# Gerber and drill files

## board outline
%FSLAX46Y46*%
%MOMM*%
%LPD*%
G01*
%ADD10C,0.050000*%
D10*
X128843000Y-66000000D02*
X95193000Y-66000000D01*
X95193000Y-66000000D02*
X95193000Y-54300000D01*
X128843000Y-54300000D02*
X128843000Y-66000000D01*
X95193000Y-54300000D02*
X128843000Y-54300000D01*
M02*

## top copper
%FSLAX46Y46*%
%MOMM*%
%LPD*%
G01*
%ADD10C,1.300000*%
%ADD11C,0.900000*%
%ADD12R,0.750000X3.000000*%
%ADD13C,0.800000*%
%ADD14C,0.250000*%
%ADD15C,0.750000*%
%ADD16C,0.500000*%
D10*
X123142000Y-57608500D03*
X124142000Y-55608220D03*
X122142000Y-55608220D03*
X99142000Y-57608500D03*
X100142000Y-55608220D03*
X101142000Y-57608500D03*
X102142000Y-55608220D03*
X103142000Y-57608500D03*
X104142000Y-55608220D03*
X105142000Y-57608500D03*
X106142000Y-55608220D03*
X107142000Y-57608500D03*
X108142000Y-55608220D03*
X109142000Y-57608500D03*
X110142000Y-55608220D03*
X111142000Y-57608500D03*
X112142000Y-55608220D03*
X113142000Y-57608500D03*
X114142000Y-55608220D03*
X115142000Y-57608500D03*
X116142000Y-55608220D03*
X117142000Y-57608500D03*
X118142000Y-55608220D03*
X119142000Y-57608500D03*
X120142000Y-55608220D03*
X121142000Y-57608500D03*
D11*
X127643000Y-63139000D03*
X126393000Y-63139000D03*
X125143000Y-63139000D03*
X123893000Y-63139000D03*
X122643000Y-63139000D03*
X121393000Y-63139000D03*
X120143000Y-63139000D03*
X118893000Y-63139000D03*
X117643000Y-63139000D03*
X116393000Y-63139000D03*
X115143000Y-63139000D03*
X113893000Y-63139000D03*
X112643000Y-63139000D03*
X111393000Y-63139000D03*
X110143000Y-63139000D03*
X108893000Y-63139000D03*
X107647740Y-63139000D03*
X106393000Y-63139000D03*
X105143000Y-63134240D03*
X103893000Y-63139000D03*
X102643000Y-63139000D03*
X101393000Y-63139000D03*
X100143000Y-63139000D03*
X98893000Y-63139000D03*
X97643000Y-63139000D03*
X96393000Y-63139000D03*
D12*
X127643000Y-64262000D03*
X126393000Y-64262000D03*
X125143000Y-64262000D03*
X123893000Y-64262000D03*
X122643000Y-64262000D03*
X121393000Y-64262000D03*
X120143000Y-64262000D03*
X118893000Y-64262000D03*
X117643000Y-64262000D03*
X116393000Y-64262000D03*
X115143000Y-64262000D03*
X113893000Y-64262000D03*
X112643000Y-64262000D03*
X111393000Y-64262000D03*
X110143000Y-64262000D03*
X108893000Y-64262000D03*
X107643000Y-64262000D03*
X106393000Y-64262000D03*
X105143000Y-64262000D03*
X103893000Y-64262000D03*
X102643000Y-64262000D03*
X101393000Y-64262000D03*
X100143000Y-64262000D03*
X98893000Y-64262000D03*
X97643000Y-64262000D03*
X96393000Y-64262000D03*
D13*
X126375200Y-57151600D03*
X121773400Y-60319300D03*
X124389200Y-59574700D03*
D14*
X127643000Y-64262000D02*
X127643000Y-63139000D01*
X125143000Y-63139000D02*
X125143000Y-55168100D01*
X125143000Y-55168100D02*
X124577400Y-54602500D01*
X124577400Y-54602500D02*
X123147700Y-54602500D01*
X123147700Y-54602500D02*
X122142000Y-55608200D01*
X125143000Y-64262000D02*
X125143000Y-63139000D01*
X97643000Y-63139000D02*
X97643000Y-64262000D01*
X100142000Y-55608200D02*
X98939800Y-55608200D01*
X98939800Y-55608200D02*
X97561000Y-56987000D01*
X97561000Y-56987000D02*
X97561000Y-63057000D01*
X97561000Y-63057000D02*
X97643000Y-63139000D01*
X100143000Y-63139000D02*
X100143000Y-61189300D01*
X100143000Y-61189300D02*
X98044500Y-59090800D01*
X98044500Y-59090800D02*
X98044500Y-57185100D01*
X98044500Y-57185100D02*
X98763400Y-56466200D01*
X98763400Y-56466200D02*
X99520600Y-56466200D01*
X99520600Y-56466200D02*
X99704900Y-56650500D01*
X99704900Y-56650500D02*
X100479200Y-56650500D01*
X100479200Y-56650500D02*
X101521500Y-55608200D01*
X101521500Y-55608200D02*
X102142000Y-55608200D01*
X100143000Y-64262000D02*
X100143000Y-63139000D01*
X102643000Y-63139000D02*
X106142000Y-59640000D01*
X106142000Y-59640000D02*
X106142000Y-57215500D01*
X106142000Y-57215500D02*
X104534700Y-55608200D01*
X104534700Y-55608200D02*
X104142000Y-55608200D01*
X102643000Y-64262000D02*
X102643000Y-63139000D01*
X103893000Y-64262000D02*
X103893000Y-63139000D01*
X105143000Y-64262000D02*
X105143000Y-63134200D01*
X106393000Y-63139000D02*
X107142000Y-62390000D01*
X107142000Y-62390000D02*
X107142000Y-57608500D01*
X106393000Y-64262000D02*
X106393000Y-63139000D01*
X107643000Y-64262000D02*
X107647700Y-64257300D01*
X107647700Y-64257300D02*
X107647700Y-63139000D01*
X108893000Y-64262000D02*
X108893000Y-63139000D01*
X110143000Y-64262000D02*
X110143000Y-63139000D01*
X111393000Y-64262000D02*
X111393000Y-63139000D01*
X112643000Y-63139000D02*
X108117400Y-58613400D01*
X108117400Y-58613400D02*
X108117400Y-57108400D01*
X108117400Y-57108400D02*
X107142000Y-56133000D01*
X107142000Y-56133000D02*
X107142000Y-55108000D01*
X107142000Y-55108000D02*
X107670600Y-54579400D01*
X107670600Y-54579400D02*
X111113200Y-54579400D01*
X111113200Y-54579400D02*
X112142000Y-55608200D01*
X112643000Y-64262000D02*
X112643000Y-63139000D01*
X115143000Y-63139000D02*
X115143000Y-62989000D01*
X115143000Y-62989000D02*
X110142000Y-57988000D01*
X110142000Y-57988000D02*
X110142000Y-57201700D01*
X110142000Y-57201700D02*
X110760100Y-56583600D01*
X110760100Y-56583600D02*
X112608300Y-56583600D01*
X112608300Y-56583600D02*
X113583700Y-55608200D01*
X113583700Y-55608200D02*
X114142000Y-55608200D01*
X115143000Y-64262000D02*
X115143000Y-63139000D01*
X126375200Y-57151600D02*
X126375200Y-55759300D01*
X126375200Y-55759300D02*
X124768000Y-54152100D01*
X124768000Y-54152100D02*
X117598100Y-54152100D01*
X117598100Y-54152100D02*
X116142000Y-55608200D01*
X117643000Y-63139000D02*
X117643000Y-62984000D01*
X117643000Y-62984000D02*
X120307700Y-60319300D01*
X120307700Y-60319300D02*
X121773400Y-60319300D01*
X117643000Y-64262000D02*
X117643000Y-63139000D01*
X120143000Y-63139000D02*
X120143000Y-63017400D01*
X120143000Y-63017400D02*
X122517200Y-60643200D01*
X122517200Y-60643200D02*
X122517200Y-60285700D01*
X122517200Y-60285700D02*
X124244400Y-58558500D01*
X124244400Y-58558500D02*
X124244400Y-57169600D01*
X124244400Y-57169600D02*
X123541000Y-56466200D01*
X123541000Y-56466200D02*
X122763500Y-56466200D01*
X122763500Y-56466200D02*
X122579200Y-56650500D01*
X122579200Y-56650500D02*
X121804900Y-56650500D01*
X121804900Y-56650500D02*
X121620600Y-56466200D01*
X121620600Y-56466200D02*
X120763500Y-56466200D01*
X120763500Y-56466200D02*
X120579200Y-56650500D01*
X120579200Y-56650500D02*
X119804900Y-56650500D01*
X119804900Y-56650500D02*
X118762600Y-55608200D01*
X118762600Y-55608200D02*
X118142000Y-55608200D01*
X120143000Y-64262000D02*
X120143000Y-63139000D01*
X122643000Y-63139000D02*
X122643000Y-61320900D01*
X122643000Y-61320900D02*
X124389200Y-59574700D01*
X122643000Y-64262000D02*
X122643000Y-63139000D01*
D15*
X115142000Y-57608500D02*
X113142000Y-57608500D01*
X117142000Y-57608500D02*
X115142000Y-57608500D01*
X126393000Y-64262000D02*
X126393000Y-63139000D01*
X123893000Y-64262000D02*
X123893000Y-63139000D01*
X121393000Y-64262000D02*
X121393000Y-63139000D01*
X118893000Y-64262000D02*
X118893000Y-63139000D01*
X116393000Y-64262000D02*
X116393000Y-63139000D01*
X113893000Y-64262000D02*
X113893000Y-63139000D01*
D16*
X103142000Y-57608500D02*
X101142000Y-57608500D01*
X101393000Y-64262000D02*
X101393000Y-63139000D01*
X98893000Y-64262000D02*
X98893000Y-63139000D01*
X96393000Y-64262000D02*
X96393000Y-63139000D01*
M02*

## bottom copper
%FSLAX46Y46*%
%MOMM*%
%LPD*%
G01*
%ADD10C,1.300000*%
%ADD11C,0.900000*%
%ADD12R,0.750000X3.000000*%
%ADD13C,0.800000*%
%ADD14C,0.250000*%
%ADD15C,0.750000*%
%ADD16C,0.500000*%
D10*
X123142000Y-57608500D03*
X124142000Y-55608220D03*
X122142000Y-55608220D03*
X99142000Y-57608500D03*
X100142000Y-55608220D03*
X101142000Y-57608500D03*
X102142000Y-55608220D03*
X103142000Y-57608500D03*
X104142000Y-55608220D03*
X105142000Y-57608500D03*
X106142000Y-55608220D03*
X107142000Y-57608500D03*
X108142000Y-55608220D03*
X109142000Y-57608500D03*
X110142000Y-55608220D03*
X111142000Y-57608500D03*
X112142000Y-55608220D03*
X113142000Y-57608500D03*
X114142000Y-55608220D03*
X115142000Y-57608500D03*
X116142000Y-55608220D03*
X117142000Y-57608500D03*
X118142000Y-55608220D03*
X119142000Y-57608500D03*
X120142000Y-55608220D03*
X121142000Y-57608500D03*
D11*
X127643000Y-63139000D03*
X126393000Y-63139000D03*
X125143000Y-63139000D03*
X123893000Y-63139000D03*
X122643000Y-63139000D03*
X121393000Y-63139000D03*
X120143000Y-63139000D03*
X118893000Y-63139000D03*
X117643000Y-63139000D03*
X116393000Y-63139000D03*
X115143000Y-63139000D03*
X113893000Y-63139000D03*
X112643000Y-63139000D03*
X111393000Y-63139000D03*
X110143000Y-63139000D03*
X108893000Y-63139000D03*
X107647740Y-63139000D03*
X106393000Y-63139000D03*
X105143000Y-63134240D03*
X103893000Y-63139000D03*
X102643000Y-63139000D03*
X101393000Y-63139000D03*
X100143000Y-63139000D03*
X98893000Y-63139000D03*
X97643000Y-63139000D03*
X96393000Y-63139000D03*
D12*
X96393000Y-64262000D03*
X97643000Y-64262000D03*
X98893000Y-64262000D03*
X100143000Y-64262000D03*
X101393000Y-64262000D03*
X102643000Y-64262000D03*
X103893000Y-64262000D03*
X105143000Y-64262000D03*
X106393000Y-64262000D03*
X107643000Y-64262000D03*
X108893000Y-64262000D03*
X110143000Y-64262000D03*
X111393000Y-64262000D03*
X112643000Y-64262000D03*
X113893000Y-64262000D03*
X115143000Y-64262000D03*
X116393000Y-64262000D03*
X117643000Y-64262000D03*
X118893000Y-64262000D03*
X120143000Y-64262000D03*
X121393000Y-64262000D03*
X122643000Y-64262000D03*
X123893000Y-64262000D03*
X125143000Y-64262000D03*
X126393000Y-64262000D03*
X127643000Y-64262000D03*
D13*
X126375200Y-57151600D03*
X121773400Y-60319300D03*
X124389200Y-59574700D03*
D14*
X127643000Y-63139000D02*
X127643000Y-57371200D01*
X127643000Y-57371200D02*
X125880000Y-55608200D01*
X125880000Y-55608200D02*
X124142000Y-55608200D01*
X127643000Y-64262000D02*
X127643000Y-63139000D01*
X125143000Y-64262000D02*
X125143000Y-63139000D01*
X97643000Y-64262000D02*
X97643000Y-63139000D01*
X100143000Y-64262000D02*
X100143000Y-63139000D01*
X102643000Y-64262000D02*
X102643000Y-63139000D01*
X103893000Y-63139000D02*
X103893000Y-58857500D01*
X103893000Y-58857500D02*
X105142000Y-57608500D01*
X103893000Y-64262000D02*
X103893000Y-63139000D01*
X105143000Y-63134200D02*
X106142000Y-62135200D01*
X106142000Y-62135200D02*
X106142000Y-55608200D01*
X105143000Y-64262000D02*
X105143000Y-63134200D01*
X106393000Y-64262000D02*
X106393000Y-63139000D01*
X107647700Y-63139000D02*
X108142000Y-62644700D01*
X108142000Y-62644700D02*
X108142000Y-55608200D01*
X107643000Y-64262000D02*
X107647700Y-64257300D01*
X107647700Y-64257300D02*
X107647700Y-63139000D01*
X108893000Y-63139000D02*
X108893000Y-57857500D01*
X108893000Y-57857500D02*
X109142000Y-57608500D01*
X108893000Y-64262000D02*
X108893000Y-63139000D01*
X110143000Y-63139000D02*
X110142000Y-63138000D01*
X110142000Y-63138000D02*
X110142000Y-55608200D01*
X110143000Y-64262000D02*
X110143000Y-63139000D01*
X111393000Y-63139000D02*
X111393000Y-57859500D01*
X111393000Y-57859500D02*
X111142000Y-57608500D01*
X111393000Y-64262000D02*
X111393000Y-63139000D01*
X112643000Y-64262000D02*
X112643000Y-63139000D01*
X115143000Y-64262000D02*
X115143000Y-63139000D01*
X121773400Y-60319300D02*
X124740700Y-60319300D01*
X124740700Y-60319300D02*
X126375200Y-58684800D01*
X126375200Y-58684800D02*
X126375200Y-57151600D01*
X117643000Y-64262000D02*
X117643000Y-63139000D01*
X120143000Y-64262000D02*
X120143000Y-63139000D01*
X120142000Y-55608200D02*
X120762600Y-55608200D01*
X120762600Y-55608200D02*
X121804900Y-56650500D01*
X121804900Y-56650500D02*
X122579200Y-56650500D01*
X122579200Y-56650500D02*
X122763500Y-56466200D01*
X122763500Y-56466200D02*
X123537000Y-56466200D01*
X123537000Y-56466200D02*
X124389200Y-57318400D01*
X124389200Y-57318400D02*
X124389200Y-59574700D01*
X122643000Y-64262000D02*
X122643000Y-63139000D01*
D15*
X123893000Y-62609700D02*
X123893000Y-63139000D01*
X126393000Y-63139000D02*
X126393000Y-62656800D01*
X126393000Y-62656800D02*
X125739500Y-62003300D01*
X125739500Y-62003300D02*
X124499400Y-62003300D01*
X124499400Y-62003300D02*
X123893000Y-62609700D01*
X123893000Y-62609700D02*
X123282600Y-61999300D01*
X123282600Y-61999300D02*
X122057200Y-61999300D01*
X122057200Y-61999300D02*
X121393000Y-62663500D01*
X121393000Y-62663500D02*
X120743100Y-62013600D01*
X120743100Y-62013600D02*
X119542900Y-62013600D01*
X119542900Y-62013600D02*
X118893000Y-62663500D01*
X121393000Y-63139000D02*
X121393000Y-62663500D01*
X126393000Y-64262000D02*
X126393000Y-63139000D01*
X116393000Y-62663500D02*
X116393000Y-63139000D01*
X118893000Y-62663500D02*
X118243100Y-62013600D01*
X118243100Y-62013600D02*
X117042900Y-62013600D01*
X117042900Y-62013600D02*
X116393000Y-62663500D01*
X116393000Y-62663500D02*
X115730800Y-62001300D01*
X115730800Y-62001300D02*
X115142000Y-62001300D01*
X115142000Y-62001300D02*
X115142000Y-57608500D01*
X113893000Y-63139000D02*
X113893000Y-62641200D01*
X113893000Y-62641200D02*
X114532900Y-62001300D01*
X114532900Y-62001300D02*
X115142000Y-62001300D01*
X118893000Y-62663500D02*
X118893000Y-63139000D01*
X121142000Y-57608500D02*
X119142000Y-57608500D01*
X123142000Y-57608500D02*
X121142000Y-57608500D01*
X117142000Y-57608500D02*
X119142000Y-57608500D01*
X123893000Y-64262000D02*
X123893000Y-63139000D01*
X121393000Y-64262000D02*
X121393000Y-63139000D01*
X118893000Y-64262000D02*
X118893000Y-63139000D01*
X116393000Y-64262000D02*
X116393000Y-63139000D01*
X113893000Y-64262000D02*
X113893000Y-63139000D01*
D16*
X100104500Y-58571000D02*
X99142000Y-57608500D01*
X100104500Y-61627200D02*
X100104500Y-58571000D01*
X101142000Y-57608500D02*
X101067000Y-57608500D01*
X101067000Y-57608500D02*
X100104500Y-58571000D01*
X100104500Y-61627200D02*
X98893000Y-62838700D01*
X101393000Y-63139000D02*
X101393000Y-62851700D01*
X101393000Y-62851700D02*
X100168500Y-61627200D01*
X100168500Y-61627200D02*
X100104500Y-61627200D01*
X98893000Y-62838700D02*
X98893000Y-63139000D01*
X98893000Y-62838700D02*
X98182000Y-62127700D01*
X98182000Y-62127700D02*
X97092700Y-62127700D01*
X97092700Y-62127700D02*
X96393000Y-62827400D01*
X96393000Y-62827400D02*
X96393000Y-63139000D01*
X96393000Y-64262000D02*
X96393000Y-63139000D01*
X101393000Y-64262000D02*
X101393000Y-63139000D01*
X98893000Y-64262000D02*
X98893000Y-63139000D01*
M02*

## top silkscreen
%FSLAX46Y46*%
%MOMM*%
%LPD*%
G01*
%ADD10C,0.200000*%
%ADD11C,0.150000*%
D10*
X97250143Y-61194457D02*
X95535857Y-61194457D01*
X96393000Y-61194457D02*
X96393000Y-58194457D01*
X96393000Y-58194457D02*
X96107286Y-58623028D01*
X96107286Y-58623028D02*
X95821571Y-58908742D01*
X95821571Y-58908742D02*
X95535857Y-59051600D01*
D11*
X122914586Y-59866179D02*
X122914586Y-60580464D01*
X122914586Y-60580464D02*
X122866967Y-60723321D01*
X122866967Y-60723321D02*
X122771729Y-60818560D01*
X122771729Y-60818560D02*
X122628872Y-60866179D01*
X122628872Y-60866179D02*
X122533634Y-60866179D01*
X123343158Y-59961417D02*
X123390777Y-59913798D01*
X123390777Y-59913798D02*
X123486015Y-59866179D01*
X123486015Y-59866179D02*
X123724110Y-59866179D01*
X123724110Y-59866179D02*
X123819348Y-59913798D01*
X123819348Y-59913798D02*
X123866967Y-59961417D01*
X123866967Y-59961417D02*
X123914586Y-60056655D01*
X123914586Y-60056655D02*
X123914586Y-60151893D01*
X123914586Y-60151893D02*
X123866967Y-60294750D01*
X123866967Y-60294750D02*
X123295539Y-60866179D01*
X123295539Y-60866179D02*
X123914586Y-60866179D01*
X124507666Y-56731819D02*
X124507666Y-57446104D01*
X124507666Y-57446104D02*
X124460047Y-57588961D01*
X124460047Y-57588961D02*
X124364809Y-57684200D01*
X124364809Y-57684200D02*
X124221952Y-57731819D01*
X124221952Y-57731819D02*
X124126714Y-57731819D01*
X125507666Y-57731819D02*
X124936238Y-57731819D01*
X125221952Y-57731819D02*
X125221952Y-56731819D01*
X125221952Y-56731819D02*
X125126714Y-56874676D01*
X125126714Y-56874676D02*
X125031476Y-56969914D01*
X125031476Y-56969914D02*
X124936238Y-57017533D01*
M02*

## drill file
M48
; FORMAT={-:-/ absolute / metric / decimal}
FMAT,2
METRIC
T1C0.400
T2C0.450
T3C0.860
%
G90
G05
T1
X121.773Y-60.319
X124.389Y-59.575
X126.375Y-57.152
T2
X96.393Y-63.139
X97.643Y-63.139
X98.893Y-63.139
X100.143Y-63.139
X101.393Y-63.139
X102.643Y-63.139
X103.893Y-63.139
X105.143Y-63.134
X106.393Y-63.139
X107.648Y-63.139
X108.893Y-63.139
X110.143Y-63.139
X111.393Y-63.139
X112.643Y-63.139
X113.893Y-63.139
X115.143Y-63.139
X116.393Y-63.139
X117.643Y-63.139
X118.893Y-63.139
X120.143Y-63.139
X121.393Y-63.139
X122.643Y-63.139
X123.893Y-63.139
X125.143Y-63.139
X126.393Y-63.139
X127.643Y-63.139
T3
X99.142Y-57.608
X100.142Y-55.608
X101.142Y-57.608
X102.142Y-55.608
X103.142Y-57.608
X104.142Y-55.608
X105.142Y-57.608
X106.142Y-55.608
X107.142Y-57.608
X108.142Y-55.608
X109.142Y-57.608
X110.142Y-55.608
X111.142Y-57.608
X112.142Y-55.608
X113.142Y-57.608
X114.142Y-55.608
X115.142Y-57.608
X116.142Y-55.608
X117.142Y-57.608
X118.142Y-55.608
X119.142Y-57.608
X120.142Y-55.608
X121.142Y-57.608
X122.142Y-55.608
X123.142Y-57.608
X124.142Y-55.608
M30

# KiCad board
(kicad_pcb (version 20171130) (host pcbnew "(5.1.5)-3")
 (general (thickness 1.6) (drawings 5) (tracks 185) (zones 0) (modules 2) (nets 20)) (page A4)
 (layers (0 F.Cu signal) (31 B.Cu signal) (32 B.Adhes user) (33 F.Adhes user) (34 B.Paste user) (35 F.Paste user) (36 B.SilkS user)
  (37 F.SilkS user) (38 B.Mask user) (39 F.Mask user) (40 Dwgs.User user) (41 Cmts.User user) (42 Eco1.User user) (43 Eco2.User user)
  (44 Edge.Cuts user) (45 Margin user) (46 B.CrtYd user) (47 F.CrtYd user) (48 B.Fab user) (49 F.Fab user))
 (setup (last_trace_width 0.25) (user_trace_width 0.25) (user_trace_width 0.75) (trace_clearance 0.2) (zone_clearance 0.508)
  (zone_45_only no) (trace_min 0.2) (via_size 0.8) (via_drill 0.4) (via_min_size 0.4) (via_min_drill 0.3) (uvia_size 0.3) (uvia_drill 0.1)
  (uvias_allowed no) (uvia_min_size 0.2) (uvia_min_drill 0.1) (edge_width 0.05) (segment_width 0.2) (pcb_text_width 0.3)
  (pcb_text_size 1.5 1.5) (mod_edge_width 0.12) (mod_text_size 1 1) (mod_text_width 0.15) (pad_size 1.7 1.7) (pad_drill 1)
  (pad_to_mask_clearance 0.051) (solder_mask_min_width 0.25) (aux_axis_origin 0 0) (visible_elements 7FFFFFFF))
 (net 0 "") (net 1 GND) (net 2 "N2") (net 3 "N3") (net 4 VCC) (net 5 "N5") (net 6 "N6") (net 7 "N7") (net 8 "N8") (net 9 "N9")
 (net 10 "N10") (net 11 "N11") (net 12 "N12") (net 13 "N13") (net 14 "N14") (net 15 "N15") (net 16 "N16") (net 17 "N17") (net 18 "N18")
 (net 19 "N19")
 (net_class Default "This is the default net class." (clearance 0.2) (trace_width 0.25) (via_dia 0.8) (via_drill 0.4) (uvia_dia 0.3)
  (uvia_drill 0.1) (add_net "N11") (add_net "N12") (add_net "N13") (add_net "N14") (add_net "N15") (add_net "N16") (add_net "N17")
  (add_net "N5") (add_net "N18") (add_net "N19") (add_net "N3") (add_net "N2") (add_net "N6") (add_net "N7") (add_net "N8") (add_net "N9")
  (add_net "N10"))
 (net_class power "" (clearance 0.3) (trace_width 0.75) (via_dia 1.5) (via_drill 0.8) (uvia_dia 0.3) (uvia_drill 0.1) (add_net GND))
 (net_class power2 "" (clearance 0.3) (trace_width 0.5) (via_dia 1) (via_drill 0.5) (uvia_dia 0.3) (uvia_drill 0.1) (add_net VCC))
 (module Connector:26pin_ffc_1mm (layer F.Cu) (at 124.142 52.8955 180)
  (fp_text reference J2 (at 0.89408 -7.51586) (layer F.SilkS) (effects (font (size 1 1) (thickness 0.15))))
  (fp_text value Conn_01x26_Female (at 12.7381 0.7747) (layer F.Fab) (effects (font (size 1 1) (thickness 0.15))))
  (pad 25 thru_hole circle (at 1 -4.713 180) (size 1.3 1.3) (drill 0.86) (layers *.Cu *.Mask) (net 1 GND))
  (pad 26 thru_hole circle (at 0 -2.71272 180) (size 1.3 1.3) (drill 0.86) (layers *.Cu *.Mask) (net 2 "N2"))
  (pad 24 thru_hole circle (at 2 -2.71272 180) (size 1.3 1.3) (drill 0.86) (layers *.Cu *.Mask) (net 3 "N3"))
  (pad 1 thru_hole circle (at 25 -4.713 180) (size 1.3 1.3) (drill 0.86) (layers *.Cu *.Mask) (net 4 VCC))
  (pad 2 thru_hole circle (at 24 -2.71272 180) (size 1.3 1.3) (drill 0.86) (layers *.Cu *.Mask) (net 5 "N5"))
  (pad 3 thru_hole circle (at 23 -4.713 180) (size 1.3 1.3) (drill 0.86) (layers *.Cu *.Mask) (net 4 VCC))
  (pad 4 thru_hole circle (at 22 -2.71272 180) (size 1.3 1.3) (drill 0.86) (layers *.Cu *.Mask) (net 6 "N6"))
  (pad 5 thru_hole circle (at 21 -4.713 180) (size 1.3 1.3) (drill 0.86) (layers *.Cu *.Mask) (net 4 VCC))
  (pad 6 thru_hole circle (at 20 -2.71272 180) (size 1.3 1.3) (drill 0.86) (layers *.Cu *.Mask) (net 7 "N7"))
  (pad 7 thru_hole circle (at 19 -4.713 180) (size 1.3 1.3) (drill 0.86) (layers *.Cu *.Mask) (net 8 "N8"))
  (pad 8 thru_hole circle (at 18 -2.71272 180) (size 1.3 1.3) (drill 0.86) (layers *.Cu *.Mask) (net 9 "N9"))
  (pad 9 thru_hole circle (at 17 -4.713 180) (size 1.3 1.3) (drill 0.86) (layers *.Cu *.Mask) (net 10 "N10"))
  (pad 10 thru_hole circle (at 16 -2.71272 180) (size 1.3 1.3) (drill 0.86) (layers *.Cu *.Mask) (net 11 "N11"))
  (pad 11 thru_hole circle (at 15 -4.713 180) (size 1.3 1.3) (drill 0.86) (layers *.Cu *.Mask) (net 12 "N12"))
  (pad 12 thru_hole circle (at 14 -2.71272 180) (size 1.3 1.3) (drill 0.86) (layers *.Cu *.Mask) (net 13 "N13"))
  (pad 13 thru_hole circle (at 13 -4.713 180) (size 1.3 1.3) (drill 0.86) (layers *.Cu *.Mask) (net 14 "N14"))
  (pad 14 thru_hole circle (at 12 -2.71272 180) (size 1.3 1.3) (drill 0.86) (layers *.Cu *.Mask) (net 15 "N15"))
  (pad 15 thru_hole circle (at 11 -4.713 180) (size 1.3 1.3) (drill 0.86) (layers *.Cu *.Mask) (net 1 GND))
  (pad 16 thru_hole circle (at 10 -2.71272 180) (size 1.3 1.3) (drill 0.86) (layers *.Cu *.Mask) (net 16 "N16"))
  (pad 17 thru_hole circle (at 9 -4.713 180) (size 1.3 1.3) (drill 0.86) (layers *.Cu *.Mask) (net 1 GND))
  (pad 18 thru_hole circle (at 8 -2.71272 180) (size 1.3 1.3) (drill 0.86) (layers *.Cu *.Mask) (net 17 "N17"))
  (pad 19 thru_hole circle (at 7 -4.713 180) (size 1.3 1.3) (drill 0.86) (layers *.Cu *.Mask) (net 1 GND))
  (pad 20 thru_hole circle (at 6 -2.71272 180) (size 1.3 1.3) (drill 0.86) (layers *.Cu *.Mask) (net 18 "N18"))
  (pad 21 thru_hole circle (at 5 -4.713 180) (size 1.3 1.3) (drill 0.86) (layers *.Cu *.Mask) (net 1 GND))
  (pad 22 thru_hole circle (at 4 -2.71272 180) (size 1.3 1.3) (drill 0.86) (layers *.Cu *.Mask) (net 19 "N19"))
  (pad 23 thru_hole circle (at 3 -4.713 180) (size 1.3 1.3) (drill 0.86) (layers *.Cu *.Mask) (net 1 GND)))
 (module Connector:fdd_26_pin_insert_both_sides (layer F.Cu) (at 96.393 64.389)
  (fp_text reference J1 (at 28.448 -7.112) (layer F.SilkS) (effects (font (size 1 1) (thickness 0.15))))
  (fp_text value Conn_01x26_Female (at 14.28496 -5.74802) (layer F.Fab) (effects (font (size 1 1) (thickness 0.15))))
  (pad 26 thru_hole circle (at 31.25 -1.25) (size 0.9 0.9) (drill 0.45) (layers *.Cu *.Mask) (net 2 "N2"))
  (pad 25 thru_hole circle (at 30 -1.25) (size 0.9 0.9) (drill 0.45) (layers *.Cu *.Mask) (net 1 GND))
  (pad 24 thru_hole circle (at 28.75 -1.25) (size 0.9 0.9) (drill 0.45) (layers *.Cu *.Mask) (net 3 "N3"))
  (pad 23 thru_hole circle (at 27.5 -1.25) (size 0.9 0.9) (drill 0.45) (layers *.Cu *.Mask) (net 1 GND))
  (pad 22 thru_hole circle (at 26.25 -1.25) (size 0.9 0.9) (drill 0.45) (layers *.Cu *.Mask) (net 19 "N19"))
  (pad 21 thru_hole circle (at 25 -1.25) (size 0.9 0.9) (drill 0.45) (layers *.Cu *.Mask) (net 1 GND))
  (pad 20 thru_hole circle (at 23.75 -1.25) (size 0.9 0.9) (drill 0.45) (layers *.Cu *.Mask) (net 18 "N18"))
  (pad 19 thru_hole circle (at 22.5 -1.25) (size 0.9 0.9) (drill 0.45) (layers *.Cu *.Mask) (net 1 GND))
  (pad 18 thru_hole circle (at 21.25 -1.25) (size 0.9 0.9) (drill 0.45) (layers *.Cu *.Mask) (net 17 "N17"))
  (pad 17 thru_hole circle (at 20 -1.25) (size 0.9 0.9) (drill 0.45) (layers *.Cu *.Mask) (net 1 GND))
  (pad 16 thru_hole circle (at 18.75 -1.25) (size 0.9 0.9) (drill 0.45) (layers *.Cu *.Mask) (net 16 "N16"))
  (pad 15 thru_hole circle (at 17.5 -1.25 90) (size 0.9 0.9) (drill 0.45) (layers *.Cu *.Mask) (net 1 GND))
  (pad 14 thru_hole circle (at 16.25 -1.25) (size 0.9 0.9) (drill 0.45) (layers *.Cu *.Mask) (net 15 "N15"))
  (pad 13 thru_hole circle (at 15 -1.25) (size 0.9 0.9) (drill 0.45) (layers *.Cu *.Mask) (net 14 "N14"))
  (pad 12 thru_hole circle (at 13.75 -1.25) (size 0.9 0.9) (drill 0.45) (layers *.Cu *.Mask) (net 13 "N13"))
  (pad 11 thru_hole circle (at 12.5 -1.25) (size 0.9 0.9) (drill 0.45) (layers *.Cu *.Mask) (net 12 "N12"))
  (pad 10 thru_hole circle (at 11.25474 -1.25) (size 0.9 0.9) (drill 0.45) (layers *.Cu *.Mask) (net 11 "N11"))
  (pad 9 thru_hole circle (at 10 -1.25) (size 0.9 0.9) (drill 0.45) (layers *.Cu *.Mask) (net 10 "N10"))
  (pad 8 thru_hole circle (at 8.75 -1.25476) (size 0.9 0.9) (drill 0.45) (layers *.Cu *.Mask) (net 9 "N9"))
  (pad 7 thru_hole circle (at 7.5 -1.25) (size 0.9 0.9) (drill 0.45) (layers *.Cu *.Mask) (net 8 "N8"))
  (pad 6 thru_hole circle (at 6.25 -1.25) (size 0.9 0.9) (drill 0.45) (layers *.Cu *.Mask) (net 7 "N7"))
  (pad 5 thru_hole circle (at 5 -1.25) (size 0.9 0.9) (drill 0.45) (layers *.Cu *.Mask) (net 4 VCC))
  (pad 4 thru_hole circle (at 3.75 -1.25) (size 0.9 0.9) (drill 0.45) (layers *.Cu *.Mask) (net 6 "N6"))
  (pad 3 thru_hole circle (at 2.5 -1.25) (size 0.9 0.9) (drill 0.45) (layers *.Cu *.Mask) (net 4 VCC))
  (pad 2 thru_hole circle (at 1.25 -1.25 90) (size 0.9 0.9) (drill 0.45) (layers *.Cu *.Mask) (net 5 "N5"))
  (pad 1 thru_hole circle (at 0 -1.25) (size 0.9 0.9) (drill 0.45) (layers *.Cu *.Mask) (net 4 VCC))
  (pad 26 connect rect (at 31.25 -0.127) (size 0.75 3) (layers F.Cu B.Mask) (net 2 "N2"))
  (pad 25 connect rect (at 30 -0.127) (size 0.75 3) (layers F.Cu B.Mask) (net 1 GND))
  (pad 24 connect rect (at 28.75 -0.127) (size 0.75 3) (layers F.Cu B.Mask) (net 3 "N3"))
  (pad 23 connect rect (at 27.5 -0.127) (size 0.75 3) (layers F.Cu B.Mask) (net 1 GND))
  (pad 22 connect rect (at 26.25 -0.127) (size 0.75 3) (layers F.Cu B.Mask) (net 19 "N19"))
  (pad 21 connect rect (at 25 -0.127) (size 0.75 3) (layers F.Cu B.Mask) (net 1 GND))
  (pad 20 connect rect (at 23.75 -0.127) (size 0.75 3) (layers F.Cu B.Mask) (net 18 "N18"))
  (pad 19 connect rect (at 22.5 -0.127) (size 0.75 3) (layers F.Cu B.Mask) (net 1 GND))
  (pad 18 connect rect (at 21.25 -0.127) (size 0.75 3) (layers F.Cu B.Mask) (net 17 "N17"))
  (pad 17 connect rect (at 20 -0.127) (size 0.75 3) (layers F.Cu B.Mask) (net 1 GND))
  (pad 16 connect rect (at 18.75 -0.127) (size 0.75 3) (layers F.Cu B.Mask) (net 16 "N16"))
  (pad 15 connect rect (at 17.5 -0.127) (size 0.75 3) (layers F.Cu B.Mask) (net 1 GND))
  (pad 14 connect rect (at 16.25 -0.127) (size 0.75 3) (layers F.Cu B.Mask) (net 15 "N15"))
  (pad 13 connect rect (at 15 -0.127) (size 0.75 3) (layers F.Cu B.Mask) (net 14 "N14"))
  (pad 12 connect rect (at 13.75 -0.127) (size 0.75 3) (layers F.Cu B.Mask) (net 13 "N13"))
  (pad 11 connect rect (at 12.5 -0.127) (size 0.75 3) (layers F.Cu B.Mask) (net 12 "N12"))
  (pad 10 connect rect (at 11.25 -0.127) (size 0.75 3) (layers F.Cu B.Mask) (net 11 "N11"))
  (pad 9 connect rect (at 10 -0.127) (size 0.75 3) (layers F.Cu B.Mask) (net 10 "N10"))
  (pad 8 connect rect (at 8.75 -0.127) (size 0.75 3) (layers F.Cu B.Mask) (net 9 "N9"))
  (pad 7 connect rect (at 7.5 -0.127) (size 0.75 3) (layers F.Cu B.Mask) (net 8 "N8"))
  (pad 6 connect rect (at 6.25 -0.127) (size 0.75 3) (layers F.Cu B.Mask) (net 7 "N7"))
  (pad 5 connect rect (at 5 -0.127) (size 0.75 3) (layers F.Cu B.Mask) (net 4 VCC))
  (pad 4 connect rect (at 3.75 -0.127) (size 0.75 3) (layers F.Cu B.Mask) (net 6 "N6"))
  (pad 3 connect rect (at 2.5 -0.127) (size 0.75 3) (layers F.Cu B.Mask) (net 4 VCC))
  (pad 2 connect rect (at 1.25 -0.127) (size 0.75 3) (layers F.Cu B.Mask) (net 5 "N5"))
  (pad 1 connect rect (at 0 -0.127) (size 0.75 3) (layers F.Cu B.Mask) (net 4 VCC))
  (pad 1 connect rect (at 0 -0.127) (size 0.75 3) (layers B.Cu B.Mask) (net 4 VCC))
  (pad 2 connect rect (at 1.25 -0.127) (size 0.75 3) (layers B.Cu B.Mask) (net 5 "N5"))
  (pad 3 connect rect (at 2.5 -0.127) (size 0.75 3) (layers B.Cu B.Mask) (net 4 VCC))
  (pad 4 connect rect (at 3.75 -0.127) (size 0.75 3) (layers B.Cu B.Mask) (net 6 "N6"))
  (pad 5 connect rect (at 5 -0.127) (size 0.75 3) (layers B.Cu B.Mask) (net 4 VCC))
  (pad 6 connect rect (at 6.25 -0.127) (size 0.75 3) (layers B.Cu B.Mask) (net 7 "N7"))
  (pad 7 connect rect (at 7.5 -0.127) (size 0.75 3) (layers B.Cu B.Mask) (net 8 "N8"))
  (pad 8 connect rect (at 8.75 -0.127) (size 0.75 3) (layers B.Cu B.Mask) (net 9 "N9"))
  (pad 9 connect rect (at 10 -0.127) (size 0.75 3) (layers B.Cu B.Mask) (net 10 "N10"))
  (pad 10 connect rect (at 11.25 -0.127) (size 0.75 3) (layers B.Cu B.Mask) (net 11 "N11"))
  (pad 11 connect rect (at 12.5 -0.127) (size 0.75 3) (layers B.Cu B.Mask) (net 12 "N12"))
  (pad 12 connect rect (at 13.75 -0.127) (size 0.75 3) (layers B.Cu B.Mask) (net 13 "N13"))
  (pad 13 connect rect (at 15 -0.127) (size 0.75 3) (layers B.Cu B.Mask) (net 14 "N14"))
  (pad 14 connect rect (at 16.25 -0.127) (size 0.75 3) (layers B.Cu B.Mask) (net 15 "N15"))
  (pad 15 connect rect (at 17.5 -0.127) (size 0.75 3) (layers B.Cu B.Mask) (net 1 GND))
  (pad 16 connect rect (at 18.75 -0.127) (size 0.75 3) (layers B.Cu B.Mask) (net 16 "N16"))
  (pad 17 connect rect (at 20 -0.127) (size 0.75 3) (layers B.Cu B.Mask) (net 1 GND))
  (pad 18 connect rect (at 21.25 -0.127) (size 0.75 3) (layers B.Cu B.Mask) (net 17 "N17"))
  (pad 19 connect rect (at 22.5 -0.127) (size 0.75 3) (layers B.Cu B.Mask) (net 1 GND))
  (pad 20 connect rect (at 23.75 -0.127) (size 0.75 3) (layers B.Cu B.Mask) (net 18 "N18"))
  (pad 21 connect rect (at 25 -0.127) (size 0.75 3) (layers B.Cu B.Mask) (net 1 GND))
  (pad 22 connect rect (at 26.25 -0.127) (size 0.75 3) (layers B.Cu B.Mask) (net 19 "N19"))
  (pad 23 connect rect (at 27.5 -0.127) (size 0.75 3) (layers B.Cu B.Mask) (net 1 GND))
  (pad 24 connect rect (at 28.75 -0.127) (size 0.75 3) (layers B.Cu B.Mask) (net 3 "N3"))
  (pad 25 connect rect (at 30 -0.127) (size 0.75 3) (layers B.Cu B.Mask) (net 1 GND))
  (pad 26 connect rect (at 31.25 -0.127) (size 0.75 3) (layers B.Cu B.Mask) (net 2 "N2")))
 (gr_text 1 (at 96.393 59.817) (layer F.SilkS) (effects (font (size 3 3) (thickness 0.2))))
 (gr_line (start 128.843 66) (end 95.193 66) (layer Edge.Cuts) (width 0.05))
 (gr_line (start 95.193 66) (end 95.193 54.3) (layer Edge.Cuts) (width 0.05))
 (gr_line (start 128.843 54.3) (end 128.843 66) (layer Edge.Cuts) (width 0.05))
 (gr_line (start 95.193 54.3) (end 128.843 54.3) (layer Edge.Cuts) (width 0.05))
 (segment (start 127.643 63.139) (end 127.643 57.3712) (width 0.25) (layer B.Cu) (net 2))
 (segment (start 127.643 57.3712) (end 125.88 55.6082) (width 0.25) (layer B.Cu) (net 2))
 (segment (start 125.88 55.6082) (end 124.142 55.6082) (width 0.25) (layer B.Cu) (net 2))
 (segment (start 127.643 64.262) (end 127.643 63.139) (width 0.25) (layer B.Cu) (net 2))
 (segment (start 127.643 64.262) (end 127.643 63.139) (width 0.25) (layer F.Cu) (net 2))
 (segment (start 125.143 63.139) (end 125.143 55.1681) (width 0.25) (layer F.Cu) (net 3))
 (segment (start 125.143 55.1681) (end 124.5774 54.6025) (width 0.25) (layer F.Cu) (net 3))
 (segment (start 124.5774 54.6025) (end 123.1477 54.6025) (width 0.25) (layer F.Cu) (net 3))
 (segment (start 123.1477 54.6025) (end 122.142 55.6082) (width 0.25) (layer F.Cu) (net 3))
 (segment (start 125.143 64.262) (end 125.143 63.139) (width 0.25) (layer F.Cu) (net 3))
 (segment (start 125.143 64.262) (end 125.143 63.139) (width 0.25) (layer B.Cu) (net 3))
 (segment (start 97.643 63.139) (end 97.643 64.262) (width 0.25) (layer F.Cu) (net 5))
 (segment (start 100.142 55.6082) (end 98.9398 55.6082) (width 0.25) (layer F.Cu) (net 5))
 (segment (start 98.9398 55.6082) (end 97.561 56.987) (width 0.25) (layer F.Cu) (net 5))
 (segment (start 97.561 56.987) (end 97.561 63.057) (width 0.25) (layer F.Cu) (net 5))
 (segment (start 97.561 63.057) (end 97.643 63.139) (width 0.25) (layer F.Cu) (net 5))
 (segment (start 97.643 64.262) (end 97.643 63.139) (width 0.25) (layer B.Cu) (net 5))
 (segment (start 100.143 64.262) (end 100.143 63.139) (width 0.25) (layer B.Cu) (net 6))
 (segment (start 100.143 63.139) (end 100.143 61.1893) (width 0.25) (layer F.Cu) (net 6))
 (segment (start 100.143 61.1893) (end 98.0445 59.0908) (width 0.25) (layer F.Cu) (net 6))
 (segment (start 98.0445 59.0908) (end 98.0445 57.1851) (width 0.25) (layer F.Cu) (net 6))
 (segment (start 98.0445 57.1851) (end 98.7634 56.4662) (width 0.25) (layer F.Cu) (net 6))
 (segment (start 98.7634 56.4662) (end 99.5206 56.4662) (width 0.25) (layer F.Cu) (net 6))
 (segment (start 99.5206 56.4662) (end 99.7049 56.6505) (width 0.25) (layer F.Cu) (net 6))
 (segment (start 99.7049 56.6505) (end 100.4792 56.6505) (width 0.25) (layer F.Cu) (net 6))
 (segment (start 100.4792 56.6505) (end 101.5215 55.6082) (width 0.25) (layer F.Cu) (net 6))
 (segment (start 101.5215 55.6082) (end 102.142 55.6082) (width 0.25) (layer F.Cu) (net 6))
 (segment (start 100.143 64.262) (end 100.143 63.139) (width 0.25) (layer F.Cu) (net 6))
 (segment (start 102.643 63.139) (end 106.142 59.64) (width 0.25) (layer F.Cu) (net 7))
 (segment (start 106.142 59.64) (end 106.142 57.2155) (width 0.25) (layer F.Cu) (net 7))
 (segment (start 106.142 57.2155) (end 104.5347 55.6082) (width 0.25) (layer F.Cu) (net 7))
 (segment (start 104.5347 55.6082) (end 104.142 55.6082) (width 0.25) (layer F.Cu) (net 7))
 (segment (start 102.643 64.262) (end 102.643 63.139) (width 0.25) (layer F.Cu) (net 7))
 (segment (start 102.643 64.262) (end 102.643 63.139) (width 0.25) (layer B.Cu) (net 7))
 (segment (start 103.893 63.139) (end 103.893 58.8575) (width 0.25) (layer B.Cu) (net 8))
 (segment (start 103.893 58.8575) (end 105.142 57.6085) (width 0.25) (layer B.Cu) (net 8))
 (segment (start 103.893 64.262) (end 103.893 63.139) (width 0.25) (layer B.Cu) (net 8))
 (segment (start 103.893 64.262) (end 103.893 63.139) (width 0.25) (layer F.Cu) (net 8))
 (segment (start 105.143 63.1342) (end 106.142 62.1352) (width 0.25) (layer B.Cu) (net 9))
 (segment (start 106.142 62.1352) (end 106.142 55.6082) (width 0.25) (layer B.Cu) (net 9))
 (segment (start 105.143 64.262) (end 105.143 63.1342) (width 0.25) (layer B.Cu) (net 9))
 (segment (start 105.143 64.262) (end 105.143 63.1342) (width 0.25) (layer F.Cu) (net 9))
 (segment (start 106.393 63.139) (end 107.142 62.39) (width 0.25) (layer F.Cu) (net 10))
 (segment (start 107.142 62.39) (end 107.142 57.6085) (width 0.25) (layer F.Cu) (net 10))
 (segment (start 106.393 64.262) (end 106.393 63.139) (width 0.25) (layer F.Cu) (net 10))
 (segment (start 106.393 64.262) (end 106.393 63.139) (width 0.25) (layer B.Cu) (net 10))
 (segment (start 107.6477 63.139) (end 108.142 62.6447) (width 0.25) (layer B.Cu) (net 11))
 (segment (start 108.142 62.6447) (end 108.142 55.6082) (width 0.25) (layer B.Cu) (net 11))
 (segment (start 107.643 64.262) (end 107.6477 64.2573) (width 0.25) (layer B.Cu) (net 11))
 (segment (start 107.6477 64.2573) (end 107.6477 63.139) (width 0.25) (layer B.Cu) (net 11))
 (segment (start 107.643 64.262) (end 107.6477 64.2573) (width 0.25) (layer F.Cu) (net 11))
 (segment (start 107.6477 64.2573) (end 107.6477 63.139) (width 0.25) (layer F.Cu) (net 11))
 (segment (start 108.893 63.139) (end 108.893 57.8575) (width 0.25) (layer B.Cu) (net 12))
 (segment (start 108.893 57.8575) (end 109.142 57.6085) (width 0.25) (layer B.Cu) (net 12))
 (segment (start 108.893 64.262) (end 108.893 63.139) (width 0.25) (layer B.Cu) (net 12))
 (segment (start 108.893 64.262) (end 108.893 63.139) (width 0.25) (layer F.Cu) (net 12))
 (segment (start 110.143 63.139) (end 110.142 63.138) (width 0.25) (layer B.Cu) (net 13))
 (segment (start 110.142 63.138) (end 110.142 55.6082) (width 0.25) (layer B.Cu) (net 13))
 (segment (start 110.143 64.262) (end 110.143 63.139) (width 0.25) (layer B.Cu) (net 13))
 (segment (start 110.143 64.262) (end 110.143 63.139) (width 0.25) (layer F.Cu) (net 13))
 (segment (start 111.393 63.139) (end 111.393 57.8595) (width 0.25) (layer B.Cu) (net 14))
 (segment (start 111.393 57.8595) (end 111.142 57.6085) (width 0.25) (layer B.Cu) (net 14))
 (segment (start 111.393 64.262) (end 111.393 63.139) (width 0.25) (layer B.Cu) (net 14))
 (segment (start 111.393 64.262) (end 111.393 63.139) (width 0.25) (layer F.Cu) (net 14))
 (segment (start 112.643 63.139) (end 108.1174 58.6134) (width 0.25) (layer F.Cu) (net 15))
 (segment (start 108.1174 58.6134) (end 108.1174 57.1084) (width 0.25) (layer F.Cu) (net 15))
 (segment (start 108.1174 57.1084) (end 107.142 56.133) (width 0.25) (layer F.Cu) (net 15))
 (segment (start 107.142 56.133) (end 107.142 55.108) (width 0.25) (layer F.Cu) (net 15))
 (segment (start 107.142 55.108) (end 107.6706 54.5794) (width 0.25) (layer F.Cu) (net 15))
 (segment (start 107.6706 54.5794) (end 111.1132 54.5794) (width 0.25) (layer F.Cu) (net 15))
 (segment (start 111.1132 54.5794) (end 112.142 55.6082) (width 0.25) (layer F.Cu) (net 15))
 (segment (start 112.643 64.262) (end 112.643 63.139) (width 0.25) (layer F.Cu) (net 15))
 (segment (start 112.643 64.262) (end 112.643 63.139) (width 0.25) (layer B.Cu) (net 15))
 (segment (start 115.143 63.139) (end 115.143 62.989) (width 0.25) (layer F.Cu) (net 16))
 (segment (start 115.143 62.989) (end 110.142 57.988) (width 0.25) (layer F.Cu) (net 16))
 (segment (start 110.142 57.988) (end 110.142 57.2017) (width 0.25) (layer F.Cu) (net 16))
 (segment (start 110.142 57.2017) (end 110.7601 56.5836) (width 0.25) (layer F.Cu) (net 16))
 (segment (start 110.7601 56.5836) (end 112.6083 56.5836) (width 0.25) (layer F.Cu) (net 16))
 (segment (start 112.6083 56.5836) (end 113.5837 55.6082) (width 0.25) (layer F.Cu) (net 16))
 (segment (start 113.5837 55.6082) (end 114.142 55.6082) (width 0.25) (layer F.Cu) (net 16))
 (segment (start 115.143 64.262) (end 115.143 63.139) (width 0.25) (layer F.Cu) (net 16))
 (segment (start 115.143 64.262) (end 115.143 63.139) (width 0.25) (layer B.Cu) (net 16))
 (segment (start 126.3752 57.1516) (end 126.3752 55.7593) (width 0.25) (layer F.Cu) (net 17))
 (segment (start 126.3752 55.7593) (end 124.768 54.1521) (width 0.25) (layer F.Cu) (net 17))
 (segment (start 124.768 54.1521) (end 117.5981 54.1521) (width 0.25) (layer F.Cu) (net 17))
 (segment (start 117.5981 54.1521) (end 116.142 55.6082) (width 0.25) (layer F.Cu) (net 17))
 (segment (start 121.7734 60.3193) (end 124.7407 60.3193) (width 0.25) (layer B.Cu) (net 17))
 (segment (start 124.7407 60.3193) (end 126.3752 58.6848) (width 0.25) (layer B.Cu) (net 17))
 (segment (start 126.3752 58.6848) (end 126.3752 57.1516) (width 0.25) (layer B.Cu) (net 17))
 (segment (start 117.643 63.139) (end 117.643 62.984) (width 0.25) (layer F.Cu) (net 17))
 (segment (start 117.643 62.984) (end 120.3077 60.3193) (width 0.25) (layer F.Cu) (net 17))
 (segment (start 120.3077 60.3193) (end 121.7734 60.3193) (width 0.25) (layer F.Cu) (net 17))
 (segment (start 117.643 64.262) (end 117.643 63.139) (width 0.25) (layer F.Cu) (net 17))
 (segment (start 117.643 64.262) (end 117.643 63.139) (width 0.25) (layer B.Cu) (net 17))
 (via (at 126.3752 57.1516) (size 0.8) (layers F.Cu B.Cu) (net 17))
 (via (at 121.7734 60.3193) (size 0.8) (layers F.Cu B.Cu) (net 17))
 (segment (start 120.143 63.139) (end 120.143 63.0174) (width 0.25) (layer F.Cu) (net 18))
 (segment (start 120.143 63.0174) (end 122.5172 60.6432) (width 0.25) (layer F.Cu) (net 18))
 (segment (start 122.5172 60.6432) (end 122.5172 60.2857) (width 0.25) (layer F.Cu) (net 18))
 (segment (start 122.5172 60.2857) (end 124.2444 58.5585) (width 0.25) (layer F.Cu) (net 18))
 (segment (start 124.2444 58.5585) (end 124.2444 57.1696) (width 0.25) (layer F.Cu) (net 18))
 (segment (start 124.2444 57.1696) (end 123.541 56.4662) (width 0.25) (layer F.Cu) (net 18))
 (segment (start 123.541 56.4662) (end 122.7635 56.4662) (width 0.25) (layer F.Cu) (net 18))
 (segment (start 122.7635 56.4662) (end 122.5792 56.6505) (width 0.25) (layer F.Cu) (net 18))
 (segment (start 122.5792 56.6505) (end 121.8049 56.6505) (width 0.25) (layer F.Cu) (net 18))
 (segment (start 121.8049 56.6505) (end 121.6206 56.4662) (width 0.25) (layer F.Cu) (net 18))
 (segment (start 121.6206 56.4662) (end 120.7635 56.4662) (width 0.25) (layer F.Cu) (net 18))
 (segment (start 120.7635 56.4662) (end 120.5792 56.6505) (width 0.25) (layer F.Cu) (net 18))
 (segment (start 120.5792 56.6505) (end 119.8049 56.6505) (width 0.25) (layer F.Cu) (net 18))
 (segment (start 119.8049 56.6505) (end 118.7626 55.6082) (width 0.25) (layer F.Cu) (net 18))
 (segment (start 118.7626 55.6082) (end 118.142 55.6082) (width 0.25) (layer F.Cu) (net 18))
 (segment (start 120.143 64.262) (end 120.143 63.139) (width 0.25) (layer F.Cu) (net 18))
 (segment (start 120.143 64.262) (end 120.143 63.139) (width 0.25) (layer B.Cu) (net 18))
 (segment (start 122.643 63.139) (end 122.643 61.3209) (width 0.25) (layer F.Cu) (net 19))
 (segment (start 122.643 61.3209) (end 124.3892 59.5747) (width 0.25) (layer F.Cu) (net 19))
 (segment (start 120.142 55.6082) (end 120.7626 55.6082) (width 0.25) (layer B.Cu) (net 19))
 (segment (start 120.7626 55.6082) (end 121.8049 56.6505) (width 0.25) (layer B.Cu) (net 19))
 (segment (start 121.8049 56.6505) (end 122.5792 56.6505) (width 0.25) (layer B.Cu) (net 19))
 (segment (start 122.5792 56.6505) (end 122.7635 56.4662) (width 0.25) (layer B.Cu) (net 19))
 (segment (start 122.7635 56.4662) (end 123.537 56.4662) (width 0.25) (layer B.Cu) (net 19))
 (segment (start 123.537 56.4662) (end 124.3892 57.3184) (width 0.25) (layer B.Cu) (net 19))
 (segment (start 124.3892 57.3184) (end 124.3892 59.5747) (width 0.25) (layer B.Cu) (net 19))
 (segment (start 122.643 64.262) (end 122.643 63.139) (width 0.25) (layer F.Cu) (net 19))
 (segment (start 122.643 64.262) (end 122.643 63.139) (width 0.25) (layer B.Cu) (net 19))
 (via (at 124.3892 59.5747) (size 0.8) (layers F.Cu B.Cu) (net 19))
 (segment (start 123.893 62.6097) (end 123.893 63.139) (width 0.75) (layer B.Cu) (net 1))
 (segment (start 126.393 63.139) (end 126.393 62.6568) (width 0.75) (layer B.Cu) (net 1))
 (segment (start 126.393 62.6568) (end 125.7395 62.0033) (width 0.75) (layer B.Cu) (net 1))
 (segment (start 125.7395 62.0033) (end 124.4994 62.0033) (width 0.75) (layer B.Cu) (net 1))
 (segment (start 124.4994 62.0033) (end 123.893 62.6097) (width 0.75) (layer B.Cu) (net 1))
 (segment (start 123.893 62.6097) (end 123.2826 61.9993) (width 0.75) (layer B.Cu) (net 1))
 (segment (start 123.2826 61.9993) (end 122.0572 61.9993) (width 0.75) (layer B.Cu) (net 1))
 (segment (start 122.0572 61.9993) (end 121.393 62.6635) (width 0.75) (layer B.Cu) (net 1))
 (segment (start 121.393 62.6635) (end 120.7431 62.0136) (width 0.75) (layer B.Cu) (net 1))
 (segment (start 120.7431 62.0136) (end 119.5429 62.0136) (width 0.75) (layer B.Cu) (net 1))
 (segment (start 119.5429 62.0136) (end 118.893 62.6635) (width 0.75) (layer B.Cu) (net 1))
 (segment (start 121.393 63.139) (end 121.393 62.6635) (width 0.75) (layer B.Cu) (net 1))
 (segment (start 126.393 64.262) (end 126.393 63.139) (width 0.75) (layer B.Cu) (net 1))
 (segment (start 116.393 62.6635) (end 116.393 63.139) (width 0.75) (layer B.Cu) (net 1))
 (segment (start 118.893 62.6635) (end 118.2431 62.0136) (width 0.75) (layer B.Cu) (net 1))
 (segment (start 118.2431 62.0136) (end 117.0429 62.0136) (width 0.75) (layer B.Cu) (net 1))
 (segment (start 117.0429 62.0136) (end 116.393 62.6635) (width 0.75) (layer B.Cu) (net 1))
 (segment (start 116.393 62.6635) (end 115.7308 62.0013) (width 0.75) (layer B.Cu) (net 1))
 (segment (start 115.7308 62.0013) (end 115.142 62.0013) (width 0.75) (layer B.Cu) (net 1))
 (segment (start 115.142 62.0013) (end 115.142 57.6085) (width 0.75) (layer B.Cu) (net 1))
 (segment (start 113.893 63.139) (end 113.893 62.6412) (width 0.75) (layer B.Cu) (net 1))
 (segment (start 113.893 62.6412) (end 114.5329 62.0013) (width 0.75) (layer B.Cu) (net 1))
 (segment (start 114.5329 62.0013) (end 115.142 62.0013) (width 0.75) (layer B.Cu) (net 1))
 (segment (start 118.893 62.6635) (end 118.893 63.139) (width 0.75) (layer B.Cu) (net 1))
 (segment (start 115.142 57.6085) (end 113.142 57.6085) (width 0.75) (layer F.Cu) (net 1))
 (segment (start 117.142 57.6085) (end 115.142 57.6085) (width 0.75) (layer F.Cu) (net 1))
 (segment (start 121.142 57.6085) (end 119.142 57.6085) (width 0.75) (layer B.Cu) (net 1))
 (segment (start 123.142 57.6085) (end 121.142 57.6085) (width 0.75) (layer B.Cu) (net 1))
 (segment (start 117.142 57.6085) (end 119.142 57.6085) (width 0.75) (layer B.Cu) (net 1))
 (segment (start 123.893 64.262) (end 123.893 63.139) (width 0.75) (layer B.Cu) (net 1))
 (segment (start 121.393 64.262) (end 121.393 63.139) (width 0.75) (layer B.Cu) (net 1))
 (segment (start 118.893 64.262) (end 118.893 63.139) (width 0.75) (layer B.Cu) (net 1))
 (segment (start 116.393 64.262) (end 116.393 63.139) (width 0.75) (layer B.Cu) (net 1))
 (segment (start 113.893 64.262) (end 113.893 63.139) (width 0.75) (layer B.Cu) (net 1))
 (segment (start 126.393 64.262) (end 126.393 63.139) (width 0.75) (layer F.Cu) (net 1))
 (segment (start 123.893 64.262) (end 123.893 63.139) (width 0.75) (layer F.Cu) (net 1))
 (segment (start 121.393 64.262) (end 121.393 63.139) (width 0.75) (layer F.Cu) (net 1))
 (segment (start 118.893 64.262) (end 118.893 63.139) (width 0.75) (layer F.Cu) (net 1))
 (segment (start 116.393 64.262) (end 116.393 63.139) (width 0.75) (layer F.Cu) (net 1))
 (segment (start 113.893 64.262) (end 113.893 63.139) (width 0.75) (layer F.Cu) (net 1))
 (segment (start 100.1045 58.571) (end 99.142 57.6085) (width 0.5) (layer B.Cu) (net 4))
 (segment (start 100.1045 61.6272) (end 100.1045 58.571) (width 0.5) (layer B.Cu) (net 4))
 (segment (start 101.142 57.6085) (end 101.067 57.6085) (width 0.5) (layer B.Cu) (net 4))
 (segment (start 101.067 57.6085) (end 100.1045 58.571) (width 0.5) (layer B.Cu) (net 4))
 (segment (start 100.1045 61.6272) (end 98.893 62.8387) (width 0.5) (layer B.Cu) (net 4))
 (segment (start 101.393 63.139) (end 101.393 62.8517) (width 0.5) (layer B.Cu) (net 4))
 (segment (start 101.393 62.8517) (end 100.1685 61.6272) (width 0.5) (layer B.Cu) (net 4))
 (segment (start 100.1685 61.6272) (end 100.1045 61.6272) (width 0.5) (layer B.Cu) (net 4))
 (segment (start 98.893 62.8387) (end 98.893 63.139) (width 0.5) (layer B.Cu) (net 4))
 (segment (start 98.893 62.8387) (end 98.182 62.1277) (width 0.5) (layer B.Cu) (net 4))
 (segment (start 98.182 62.1277) (end 97.0927 62.1277) (width 0.5) (layer B.Cu) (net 4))
 (segment (start 97.0927 62.1277) (end 96.393 62.8274) (width 0.5) (layer B.Cu) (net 4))
 (segment (start 96.393 62.8274) (end 96.393 63.139) (width 0.5) (layer B.Cu) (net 4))
 (segment (start 96.393 64.262) (end 96.393 63.139) (width 0.5) (layer B.Cu) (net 4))
 (segment (start 101.393 64.262) (end 101.393 63.139) (width 0.5) (layer B.Cu) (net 4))
 (segment (start 103.142 57.6085) (end 101.142 57.6085) (width 0.5) (layer F.Cu) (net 4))
 (segment (start 98.893 64.262) (end 98.893 63.139) (width 0.5) (layer B.Cu) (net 4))
 (segment (start 101.393 64.262) (end 101.393 63.139) (width 0.5) (layer F.Cu) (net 4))
 (segment (start 98.893 64.262) (end 98.893 63.139) (width 0.5) (layer F.Cu) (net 4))
 (segment (start 96.393 64.262) (end 96.393 63.139) (width 0.5) (layer F.Cu) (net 4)))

